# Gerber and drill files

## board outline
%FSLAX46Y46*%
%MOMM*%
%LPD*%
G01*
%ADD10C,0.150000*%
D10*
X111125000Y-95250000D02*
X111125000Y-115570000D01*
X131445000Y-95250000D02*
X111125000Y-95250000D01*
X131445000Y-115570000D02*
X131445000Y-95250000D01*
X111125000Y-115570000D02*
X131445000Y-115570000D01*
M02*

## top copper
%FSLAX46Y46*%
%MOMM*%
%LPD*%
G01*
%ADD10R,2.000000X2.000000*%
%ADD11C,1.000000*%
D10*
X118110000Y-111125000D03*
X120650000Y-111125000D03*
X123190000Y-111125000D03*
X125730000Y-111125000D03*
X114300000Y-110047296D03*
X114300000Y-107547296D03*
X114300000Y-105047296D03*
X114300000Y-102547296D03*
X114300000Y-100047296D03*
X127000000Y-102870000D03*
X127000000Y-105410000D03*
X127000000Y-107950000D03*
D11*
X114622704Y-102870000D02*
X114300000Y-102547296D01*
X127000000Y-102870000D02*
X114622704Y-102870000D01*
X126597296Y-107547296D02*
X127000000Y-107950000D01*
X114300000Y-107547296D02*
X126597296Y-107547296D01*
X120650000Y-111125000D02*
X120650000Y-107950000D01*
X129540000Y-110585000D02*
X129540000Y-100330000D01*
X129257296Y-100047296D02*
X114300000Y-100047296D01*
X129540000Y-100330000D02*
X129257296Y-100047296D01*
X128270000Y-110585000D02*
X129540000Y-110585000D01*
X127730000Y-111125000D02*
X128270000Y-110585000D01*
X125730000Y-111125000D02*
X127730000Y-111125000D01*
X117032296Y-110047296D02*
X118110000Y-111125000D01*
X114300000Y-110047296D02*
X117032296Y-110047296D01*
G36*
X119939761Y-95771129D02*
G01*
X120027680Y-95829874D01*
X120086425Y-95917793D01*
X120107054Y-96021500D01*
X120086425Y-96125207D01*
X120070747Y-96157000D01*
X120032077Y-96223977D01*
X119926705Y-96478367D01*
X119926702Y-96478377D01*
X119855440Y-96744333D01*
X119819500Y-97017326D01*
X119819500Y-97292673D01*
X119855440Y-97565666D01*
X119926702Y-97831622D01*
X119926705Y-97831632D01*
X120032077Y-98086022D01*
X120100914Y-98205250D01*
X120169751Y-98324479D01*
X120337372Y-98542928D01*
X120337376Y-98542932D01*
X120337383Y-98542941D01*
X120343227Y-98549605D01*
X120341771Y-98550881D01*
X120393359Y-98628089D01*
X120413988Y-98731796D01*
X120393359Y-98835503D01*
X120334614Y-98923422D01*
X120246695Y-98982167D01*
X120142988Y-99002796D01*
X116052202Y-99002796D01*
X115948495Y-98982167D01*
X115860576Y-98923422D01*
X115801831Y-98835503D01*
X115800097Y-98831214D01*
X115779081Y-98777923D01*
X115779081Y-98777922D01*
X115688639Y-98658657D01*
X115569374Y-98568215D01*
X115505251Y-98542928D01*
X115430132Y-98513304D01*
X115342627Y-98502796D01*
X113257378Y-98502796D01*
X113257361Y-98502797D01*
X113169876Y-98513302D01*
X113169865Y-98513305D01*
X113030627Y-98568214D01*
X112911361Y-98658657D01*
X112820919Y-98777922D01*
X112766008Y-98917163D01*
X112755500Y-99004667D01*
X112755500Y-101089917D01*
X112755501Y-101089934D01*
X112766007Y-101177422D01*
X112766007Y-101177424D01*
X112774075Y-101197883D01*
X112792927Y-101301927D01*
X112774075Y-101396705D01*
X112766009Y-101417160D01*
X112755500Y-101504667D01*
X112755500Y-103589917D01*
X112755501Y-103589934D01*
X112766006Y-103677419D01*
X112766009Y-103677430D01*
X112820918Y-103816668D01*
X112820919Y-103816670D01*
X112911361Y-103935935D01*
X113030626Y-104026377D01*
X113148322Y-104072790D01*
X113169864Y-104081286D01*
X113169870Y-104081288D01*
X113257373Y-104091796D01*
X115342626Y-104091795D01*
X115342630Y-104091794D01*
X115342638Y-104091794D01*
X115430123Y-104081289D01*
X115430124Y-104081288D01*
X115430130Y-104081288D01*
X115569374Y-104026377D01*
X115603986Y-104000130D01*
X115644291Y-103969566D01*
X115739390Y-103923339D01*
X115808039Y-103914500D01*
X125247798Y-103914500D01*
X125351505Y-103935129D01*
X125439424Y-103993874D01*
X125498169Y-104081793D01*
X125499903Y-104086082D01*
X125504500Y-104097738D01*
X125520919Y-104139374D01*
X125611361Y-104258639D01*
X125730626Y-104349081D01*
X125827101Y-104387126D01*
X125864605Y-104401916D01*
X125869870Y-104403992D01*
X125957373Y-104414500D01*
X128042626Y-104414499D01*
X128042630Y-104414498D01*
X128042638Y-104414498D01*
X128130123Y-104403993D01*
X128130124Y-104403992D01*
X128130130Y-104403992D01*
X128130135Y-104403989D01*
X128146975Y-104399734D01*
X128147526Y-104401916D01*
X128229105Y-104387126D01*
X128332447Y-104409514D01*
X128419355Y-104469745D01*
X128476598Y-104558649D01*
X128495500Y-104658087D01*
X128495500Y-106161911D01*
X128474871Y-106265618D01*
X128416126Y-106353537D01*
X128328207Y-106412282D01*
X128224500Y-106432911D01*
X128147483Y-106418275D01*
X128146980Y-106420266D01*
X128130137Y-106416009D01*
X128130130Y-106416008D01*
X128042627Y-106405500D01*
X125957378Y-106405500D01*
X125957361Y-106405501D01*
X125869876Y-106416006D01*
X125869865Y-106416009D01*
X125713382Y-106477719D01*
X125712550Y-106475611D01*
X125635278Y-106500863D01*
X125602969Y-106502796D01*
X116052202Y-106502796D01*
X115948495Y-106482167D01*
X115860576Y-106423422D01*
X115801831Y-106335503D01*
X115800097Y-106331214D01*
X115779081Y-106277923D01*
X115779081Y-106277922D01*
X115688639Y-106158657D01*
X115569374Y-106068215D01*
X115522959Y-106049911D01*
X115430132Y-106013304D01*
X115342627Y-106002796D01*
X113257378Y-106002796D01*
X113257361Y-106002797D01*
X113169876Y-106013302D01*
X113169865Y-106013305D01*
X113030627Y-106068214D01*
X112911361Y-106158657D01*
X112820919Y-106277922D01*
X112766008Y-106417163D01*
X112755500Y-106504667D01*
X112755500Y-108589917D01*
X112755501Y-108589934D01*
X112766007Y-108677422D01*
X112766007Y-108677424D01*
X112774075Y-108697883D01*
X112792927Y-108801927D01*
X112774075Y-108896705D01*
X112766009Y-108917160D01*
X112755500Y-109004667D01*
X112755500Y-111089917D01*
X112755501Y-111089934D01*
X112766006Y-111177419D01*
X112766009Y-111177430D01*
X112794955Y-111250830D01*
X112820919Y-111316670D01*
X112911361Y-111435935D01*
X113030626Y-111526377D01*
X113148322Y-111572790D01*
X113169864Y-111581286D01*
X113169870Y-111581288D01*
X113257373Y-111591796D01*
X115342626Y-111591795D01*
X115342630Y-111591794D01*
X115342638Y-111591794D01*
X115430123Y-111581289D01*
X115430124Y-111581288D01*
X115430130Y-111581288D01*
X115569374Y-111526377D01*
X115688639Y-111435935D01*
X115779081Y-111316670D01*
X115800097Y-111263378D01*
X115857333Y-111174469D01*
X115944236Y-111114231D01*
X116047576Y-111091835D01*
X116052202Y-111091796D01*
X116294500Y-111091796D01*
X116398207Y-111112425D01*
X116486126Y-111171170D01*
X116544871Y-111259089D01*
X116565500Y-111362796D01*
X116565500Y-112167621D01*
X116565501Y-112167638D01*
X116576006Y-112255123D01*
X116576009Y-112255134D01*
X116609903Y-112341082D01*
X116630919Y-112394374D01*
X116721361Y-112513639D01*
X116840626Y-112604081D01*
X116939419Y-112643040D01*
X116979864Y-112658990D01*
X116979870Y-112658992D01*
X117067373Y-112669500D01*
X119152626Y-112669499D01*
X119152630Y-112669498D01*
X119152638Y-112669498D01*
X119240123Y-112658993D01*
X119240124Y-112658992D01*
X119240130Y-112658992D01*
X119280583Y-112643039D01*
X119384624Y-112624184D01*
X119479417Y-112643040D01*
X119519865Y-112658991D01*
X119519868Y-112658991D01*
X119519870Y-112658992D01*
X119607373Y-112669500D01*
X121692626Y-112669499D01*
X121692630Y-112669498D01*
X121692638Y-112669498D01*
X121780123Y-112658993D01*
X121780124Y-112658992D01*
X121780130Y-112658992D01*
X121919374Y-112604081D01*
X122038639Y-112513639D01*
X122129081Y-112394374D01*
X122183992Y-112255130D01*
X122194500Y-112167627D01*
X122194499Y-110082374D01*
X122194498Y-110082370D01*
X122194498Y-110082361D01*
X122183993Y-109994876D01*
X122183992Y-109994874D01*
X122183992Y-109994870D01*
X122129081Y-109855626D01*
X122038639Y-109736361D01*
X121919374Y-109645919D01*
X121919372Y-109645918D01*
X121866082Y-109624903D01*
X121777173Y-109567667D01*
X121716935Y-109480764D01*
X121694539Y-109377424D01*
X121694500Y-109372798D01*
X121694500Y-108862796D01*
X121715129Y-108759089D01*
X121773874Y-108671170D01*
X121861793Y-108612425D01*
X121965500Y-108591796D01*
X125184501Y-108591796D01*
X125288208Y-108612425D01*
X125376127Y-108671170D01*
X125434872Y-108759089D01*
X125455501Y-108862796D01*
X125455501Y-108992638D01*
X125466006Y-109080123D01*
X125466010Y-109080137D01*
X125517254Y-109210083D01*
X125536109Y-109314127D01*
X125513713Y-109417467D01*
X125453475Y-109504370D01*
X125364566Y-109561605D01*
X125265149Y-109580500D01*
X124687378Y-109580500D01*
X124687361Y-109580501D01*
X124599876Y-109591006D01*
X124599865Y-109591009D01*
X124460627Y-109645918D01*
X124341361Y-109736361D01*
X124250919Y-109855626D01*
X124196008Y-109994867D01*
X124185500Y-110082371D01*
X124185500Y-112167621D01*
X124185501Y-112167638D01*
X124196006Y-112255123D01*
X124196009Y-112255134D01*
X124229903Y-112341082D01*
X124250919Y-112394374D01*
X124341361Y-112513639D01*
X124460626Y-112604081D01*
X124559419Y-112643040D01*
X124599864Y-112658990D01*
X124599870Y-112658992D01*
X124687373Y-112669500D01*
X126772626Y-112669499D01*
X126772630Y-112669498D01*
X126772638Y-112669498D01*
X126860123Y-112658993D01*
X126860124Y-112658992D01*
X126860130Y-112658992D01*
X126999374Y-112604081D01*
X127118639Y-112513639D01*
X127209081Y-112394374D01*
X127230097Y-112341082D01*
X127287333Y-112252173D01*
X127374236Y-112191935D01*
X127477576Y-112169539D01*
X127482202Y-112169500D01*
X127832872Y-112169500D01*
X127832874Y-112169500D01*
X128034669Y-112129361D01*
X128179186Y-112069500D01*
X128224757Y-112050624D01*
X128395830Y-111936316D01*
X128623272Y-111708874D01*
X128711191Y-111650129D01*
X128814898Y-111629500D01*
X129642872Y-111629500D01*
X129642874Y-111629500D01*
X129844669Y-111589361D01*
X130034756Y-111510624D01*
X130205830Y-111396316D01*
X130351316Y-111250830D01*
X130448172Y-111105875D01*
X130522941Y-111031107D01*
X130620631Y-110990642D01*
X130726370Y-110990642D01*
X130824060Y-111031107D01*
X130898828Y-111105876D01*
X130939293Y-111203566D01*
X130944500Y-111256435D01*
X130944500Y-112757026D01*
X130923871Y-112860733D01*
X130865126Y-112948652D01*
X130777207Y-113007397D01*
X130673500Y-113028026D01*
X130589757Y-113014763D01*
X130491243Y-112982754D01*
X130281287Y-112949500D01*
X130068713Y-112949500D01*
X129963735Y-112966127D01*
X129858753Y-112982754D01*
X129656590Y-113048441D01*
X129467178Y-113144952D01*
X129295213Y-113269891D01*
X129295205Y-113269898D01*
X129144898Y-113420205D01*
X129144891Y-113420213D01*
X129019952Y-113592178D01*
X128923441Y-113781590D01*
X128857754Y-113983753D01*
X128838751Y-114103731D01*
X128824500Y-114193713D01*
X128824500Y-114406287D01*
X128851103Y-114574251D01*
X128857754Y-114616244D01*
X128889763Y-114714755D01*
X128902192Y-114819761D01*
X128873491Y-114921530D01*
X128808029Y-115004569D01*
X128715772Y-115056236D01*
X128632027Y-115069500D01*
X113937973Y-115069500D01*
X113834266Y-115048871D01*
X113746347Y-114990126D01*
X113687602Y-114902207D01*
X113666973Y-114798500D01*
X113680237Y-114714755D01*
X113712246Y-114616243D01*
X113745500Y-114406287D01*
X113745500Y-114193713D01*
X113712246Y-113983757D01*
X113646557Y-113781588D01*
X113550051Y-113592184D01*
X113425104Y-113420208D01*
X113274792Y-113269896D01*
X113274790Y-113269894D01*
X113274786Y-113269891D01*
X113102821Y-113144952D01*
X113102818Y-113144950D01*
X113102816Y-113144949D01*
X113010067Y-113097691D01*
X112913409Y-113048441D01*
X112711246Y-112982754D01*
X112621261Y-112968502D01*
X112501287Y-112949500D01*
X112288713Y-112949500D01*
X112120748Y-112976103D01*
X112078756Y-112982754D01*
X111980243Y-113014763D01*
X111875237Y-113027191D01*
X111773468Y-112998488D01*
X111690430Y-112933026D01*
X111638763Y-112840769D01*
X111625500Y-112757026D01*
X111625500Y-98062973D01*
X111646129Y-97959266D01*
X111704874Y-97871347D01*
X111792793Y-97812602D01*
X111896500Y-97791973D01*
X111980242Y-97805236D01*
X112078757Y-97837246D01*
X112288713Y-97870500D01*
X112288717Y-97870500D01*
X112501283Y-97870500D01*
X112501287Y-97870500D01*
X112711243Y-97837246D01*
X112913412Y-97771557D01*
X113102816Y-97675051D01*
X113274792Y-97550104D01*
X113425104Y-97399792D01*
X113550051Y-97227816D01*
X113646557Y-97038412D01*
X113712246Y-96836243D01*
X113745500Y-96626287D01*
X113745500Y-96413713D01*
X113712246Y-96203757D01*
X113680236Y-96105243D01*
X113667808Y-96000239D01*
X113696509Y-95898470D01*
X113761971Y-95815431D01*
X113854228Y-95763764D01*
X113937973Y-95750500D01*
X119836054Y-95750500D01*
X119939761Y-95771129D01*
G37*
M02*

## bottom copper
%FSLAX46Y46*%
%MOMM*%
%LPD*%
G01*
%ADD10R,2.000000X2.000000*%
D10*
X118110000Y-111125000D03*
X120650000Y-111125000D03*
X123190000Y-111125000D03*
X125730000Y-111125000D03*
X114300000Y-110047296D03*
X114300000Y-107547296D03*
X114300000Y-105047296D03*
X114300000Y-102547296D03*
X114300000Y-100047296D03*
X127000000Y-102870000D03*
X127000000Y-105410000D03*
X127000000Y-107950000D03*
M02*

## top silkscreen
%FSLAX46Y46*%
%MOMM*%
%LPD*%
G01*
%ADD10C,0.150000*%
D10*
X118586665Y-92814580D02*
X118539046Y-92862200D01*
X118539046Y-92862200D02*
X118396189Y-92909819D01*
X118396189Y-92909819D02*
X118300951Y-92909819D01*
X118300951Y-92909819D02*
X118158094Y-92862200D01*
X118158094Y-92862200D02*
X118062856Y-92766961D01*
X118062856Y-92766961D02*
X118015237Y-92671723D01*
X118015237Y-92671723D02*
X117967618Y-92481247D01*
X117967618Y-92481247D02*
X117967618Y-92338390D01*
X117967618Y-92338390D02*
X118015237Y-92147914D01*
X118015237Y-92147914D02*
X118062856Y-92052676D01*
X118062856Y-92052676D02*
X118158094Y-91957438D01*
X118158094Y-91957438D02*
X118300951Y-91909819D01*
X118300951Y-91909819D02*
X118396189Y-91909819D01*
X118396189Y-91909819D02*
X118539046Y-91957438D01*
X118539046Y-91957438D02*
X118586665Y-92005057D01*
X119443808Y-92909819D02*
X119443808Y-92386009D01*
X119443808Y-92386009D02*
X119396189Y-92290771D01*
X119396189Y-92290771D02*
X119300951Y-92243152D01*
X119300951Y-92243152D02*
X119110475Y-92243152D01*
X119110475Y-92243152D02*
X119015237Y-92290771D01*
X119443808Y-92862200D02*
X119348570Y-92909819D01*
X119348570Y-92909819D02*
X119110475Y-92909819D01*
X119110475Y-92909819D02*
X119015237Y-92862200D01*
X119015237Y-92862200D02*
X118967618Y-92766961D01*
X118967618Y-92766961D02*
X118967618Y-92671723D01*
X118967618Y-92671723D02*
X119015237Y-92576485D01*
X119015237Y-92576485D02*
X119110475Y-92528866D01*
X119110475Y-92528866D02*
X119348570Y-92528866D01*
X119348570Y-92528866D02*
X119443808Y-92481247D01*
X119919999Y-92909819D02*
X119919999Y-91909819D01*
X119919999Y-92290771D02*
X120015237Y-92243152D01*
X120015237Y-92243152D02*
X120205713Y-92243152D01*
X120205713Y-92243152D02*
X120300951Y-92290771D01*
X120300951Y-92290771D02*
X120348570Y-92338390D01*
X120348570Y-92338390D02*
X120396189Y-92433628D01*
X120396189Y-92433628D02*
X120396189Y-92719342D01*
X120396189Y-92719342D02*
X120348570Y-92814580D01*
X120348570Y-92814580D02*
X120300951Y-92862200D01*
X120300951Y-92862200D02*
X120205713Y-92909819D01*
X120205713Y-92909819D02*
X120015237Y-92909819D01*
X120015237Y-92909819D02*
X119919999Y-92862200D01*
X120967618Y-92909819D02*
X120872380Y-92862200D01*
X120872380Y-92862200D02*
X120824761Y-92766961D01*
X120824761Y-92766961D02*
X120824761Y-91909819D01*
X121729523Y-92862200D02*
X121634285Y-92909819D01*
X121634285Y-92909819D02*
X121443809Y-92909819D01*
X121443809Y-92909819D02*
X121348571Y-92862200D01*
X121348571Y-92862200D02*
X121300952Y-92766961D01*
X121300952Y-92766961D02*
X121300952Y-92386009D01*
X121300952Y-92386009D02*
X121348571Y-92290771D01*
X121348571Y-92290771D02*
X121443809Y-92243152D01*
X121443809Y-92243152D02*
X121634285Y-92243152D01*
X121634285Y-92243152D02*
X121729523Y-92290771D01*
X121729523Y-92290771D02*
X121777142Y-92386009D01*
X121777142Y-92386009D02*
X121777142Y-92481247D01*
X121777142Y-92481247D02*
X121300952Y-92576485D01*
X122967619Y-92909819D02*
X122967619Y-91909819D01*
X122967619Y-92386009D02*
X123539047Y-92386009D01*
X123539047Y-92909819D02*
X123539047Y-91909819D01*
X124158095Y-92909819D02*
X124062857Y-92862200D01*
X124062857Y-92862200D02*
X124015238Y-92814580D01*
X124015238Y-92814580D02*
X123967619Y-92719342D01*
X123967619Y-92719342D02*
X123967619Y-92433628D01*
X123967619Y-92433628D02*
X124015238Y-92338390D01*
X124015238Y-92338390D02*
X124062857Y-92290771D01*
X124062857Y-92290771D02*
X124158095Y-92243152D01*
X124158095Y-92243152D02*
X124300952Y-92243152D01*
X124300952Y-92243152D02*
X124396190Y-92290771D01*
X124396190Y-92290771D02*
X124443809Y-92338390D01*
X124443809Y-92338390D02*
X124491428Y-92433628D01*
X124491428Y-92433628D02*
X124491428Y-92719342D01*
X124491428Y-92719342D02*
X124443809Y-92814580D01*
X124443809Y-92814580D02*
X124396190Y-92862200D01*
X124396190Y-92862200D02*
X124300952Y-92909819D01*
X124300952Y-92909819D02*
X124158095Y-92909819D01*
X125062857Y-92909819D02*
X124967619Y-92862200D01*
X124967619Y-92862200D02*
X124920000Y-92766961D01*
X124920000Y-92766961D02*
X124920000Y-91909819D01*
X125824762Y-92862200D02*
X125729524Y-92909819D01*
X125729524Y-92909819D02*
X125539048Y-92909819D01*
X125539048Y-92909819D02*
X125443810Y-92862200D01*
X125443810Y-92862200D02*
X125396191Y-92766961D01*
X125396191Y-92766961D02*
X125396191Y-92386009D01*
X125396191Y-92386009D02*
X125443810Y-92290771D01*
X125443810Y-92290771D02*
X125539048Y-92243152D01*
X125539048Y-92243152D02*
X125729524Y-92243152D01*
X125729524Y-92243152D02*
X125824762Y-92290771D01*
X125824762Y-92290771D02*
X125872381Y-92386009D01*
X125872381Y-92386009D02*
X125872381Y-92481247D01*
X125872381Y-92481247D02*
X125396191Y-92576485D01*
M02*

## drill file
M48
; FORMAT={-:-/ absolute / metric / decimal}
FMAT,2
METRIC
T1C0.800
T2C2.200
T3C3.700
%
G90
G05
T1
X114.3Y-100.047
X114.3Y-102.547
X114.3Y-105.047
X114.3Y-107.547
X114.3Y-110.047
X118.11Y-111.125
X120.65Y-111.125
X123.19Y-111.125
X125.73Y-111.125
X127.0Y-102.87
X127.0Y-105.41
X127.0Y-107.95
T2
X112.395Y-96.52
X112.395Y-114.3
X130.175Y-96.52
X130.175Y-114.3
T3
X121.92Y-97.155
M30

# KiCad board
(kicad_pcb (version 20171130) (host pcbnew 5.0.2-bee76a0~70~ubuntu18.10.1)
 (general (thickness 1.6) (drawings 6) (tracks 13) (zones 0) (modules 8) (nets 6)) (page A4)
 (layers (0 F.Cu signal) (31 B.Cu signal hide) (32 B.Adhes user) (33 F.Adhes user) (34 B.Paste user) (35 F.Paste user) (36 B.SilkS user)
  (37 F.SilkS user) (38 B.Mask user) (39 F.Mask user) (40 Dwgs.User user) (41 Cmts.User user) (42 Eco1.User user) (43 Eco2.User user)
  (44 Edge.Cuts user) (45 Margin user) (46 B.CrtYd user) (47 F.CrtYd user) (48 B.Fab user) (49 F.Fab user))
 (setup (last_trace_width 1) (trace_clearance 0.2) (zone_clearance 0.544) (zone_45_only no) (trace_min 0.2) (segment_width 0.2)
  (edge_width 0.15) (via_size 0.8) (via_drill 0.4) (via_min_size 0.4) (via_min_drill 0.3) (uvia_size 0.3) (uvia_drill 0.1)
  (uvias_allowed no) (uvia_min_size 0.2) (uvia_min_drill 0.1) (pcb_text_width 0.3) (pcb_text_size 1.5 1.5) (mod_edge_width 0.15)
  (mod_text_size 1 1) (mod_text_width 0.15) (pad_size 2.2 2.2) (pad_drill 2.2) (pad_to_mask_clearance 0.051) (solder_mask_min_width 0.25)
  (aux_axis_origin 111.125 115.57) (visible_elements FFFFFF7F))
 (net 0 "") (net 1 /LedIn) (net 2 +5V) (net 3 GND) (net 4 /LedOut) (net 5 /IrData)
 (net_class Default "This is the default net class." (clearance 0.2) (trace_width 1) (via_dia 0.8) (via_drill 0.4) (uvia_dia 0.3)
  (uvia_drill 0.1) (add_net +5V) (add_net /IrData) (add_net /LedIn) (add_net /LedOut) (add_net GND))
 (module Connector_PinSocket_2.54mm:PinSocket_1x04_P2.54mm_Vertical (layer B.Cu) (at 118.11 111.125 270)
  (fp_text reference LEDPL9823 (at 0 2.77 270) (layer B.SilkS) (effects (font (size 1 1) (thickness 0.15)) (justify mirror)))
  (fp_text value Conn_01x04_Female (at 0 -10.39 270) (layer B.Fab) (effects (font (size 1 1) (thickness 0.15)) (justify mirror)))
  (pad 1 thru_hole rect (at 0 0 270) (size 2 2) (drill 0.8) (layers *.Cu *.Mask) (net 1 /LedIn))
  (pad 2 thru_hole rect (at 0 -2.54 270) (size 2 2) (drill 0.8) (layers *.Cu *.Mask) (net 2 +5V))
  (pad 3 thru_hole rect (at 0 -5.08 270) (size 2 2) (drill 0.8) (layers *.Cu *.Mask) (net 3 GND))
  (pad 4 thru_hole rect (at 0 -7.62 270) (size 2 2) (drill 0.8) (layers *.Cu *.Mask) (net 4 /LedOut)))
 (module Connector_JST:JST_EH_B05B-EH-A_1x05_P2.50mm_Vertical (layer B.Cu) (at 114.3 110.047296 90)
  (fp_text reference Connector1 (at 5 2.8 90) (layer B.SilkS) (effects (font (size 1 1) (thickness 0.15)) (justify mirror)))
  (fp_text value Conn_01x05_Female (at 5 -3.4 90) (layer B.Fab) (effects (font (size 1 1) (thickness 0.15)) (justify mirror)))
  (pad 1 thru_hole rect (at 0 0 90) (size 2 2) (drill 0.8) (layers *.Cu *.Mask) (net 1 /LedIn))
  (pad 2 thru_hole rect (at 2.5 0 90) (size 2 2) (drill 0.8) (layers *.Cu *.Mask) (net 2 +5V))
  (pad 3 thru_hole rect (at 5 0 90) (size 2 2) (drill 0.8) (layers *.Cu *.Mask) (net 3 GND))
  (pad 4 thru_hole rect (at 7.5 0 90) (size 2 2) (drill 0.8) (layers *.Cu *.Mask) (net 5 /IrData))
  (pad 5 thru_hole rect (at 10 0 90) (size 2 2) (drill 0.8) (layers *.Cu *.Mask) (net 4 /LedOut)))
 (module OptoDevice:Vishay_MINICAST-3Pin (layer B.Cu) (at 127 102.87 270)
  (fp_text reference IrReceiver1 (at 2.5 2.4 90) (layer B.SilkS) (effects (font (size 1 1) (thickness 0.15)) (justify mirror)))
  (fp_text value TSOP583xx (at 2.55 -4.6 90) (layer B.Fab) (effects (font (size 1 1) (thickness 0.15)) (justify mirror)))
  (pad 1 thru_hole rect (at 0 0 270) (size 2 2) (drill 0.8) (layers *.Cu *.Mask) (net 5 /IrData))
  (pad 2 thru_hole rect (at 2.54 0 270) (size 2 2) (drill 0.8) (layers *.Cu *.Mask) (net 3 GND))
  (pad 3 thru_hole rect (at 5.08 0 270) (size 2 2) (drill 0.8) (layers *.Cu *.Mask) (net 2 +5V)))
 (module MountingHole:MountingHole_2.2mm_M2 (layer F.Cu) (at 112.395 96.52)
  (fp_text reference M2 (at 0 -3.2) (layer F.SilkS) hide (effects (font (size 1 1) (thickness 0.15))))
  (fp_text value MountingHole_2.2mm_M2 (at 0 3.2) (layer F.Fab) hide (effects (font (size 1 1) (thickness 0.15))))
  (pad "" np_thru_hole circle (at 0 0) (size 2.2 2.2) (drill 2.2) (layers *.Cu *.Mask)))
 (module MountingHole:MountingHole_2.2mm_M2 (layer F.Cu) (at 112.395 114.3)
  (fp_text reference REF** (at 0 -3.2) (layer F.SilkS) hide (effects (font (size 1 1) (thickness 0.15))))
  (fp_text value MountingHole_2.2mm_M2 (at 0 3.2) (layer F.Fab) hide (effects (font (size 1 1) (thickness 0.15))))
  (pad 1 np_thru_hole circle (at 0 0) (size 2.2 2.2) (drill 2.2) (layers *.Cu *.Mask)))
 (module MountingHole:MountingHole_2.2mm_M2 (layer F.Cu) (at 130.175 114.3)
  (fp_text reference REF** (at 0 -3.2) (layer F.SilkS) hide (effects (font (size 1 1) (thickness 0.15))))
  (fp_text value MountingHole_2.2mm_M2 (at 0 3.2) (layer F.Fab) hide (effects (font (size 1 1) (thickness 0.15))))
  (pad 1 np_thru_hole circle (at 0 0) (size 2.2 2.2) (drill 2.2) (layers *.Cu *.Mask)))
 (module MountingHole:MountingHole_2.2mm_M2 (layer F.Cu) (at 130.175 96.52)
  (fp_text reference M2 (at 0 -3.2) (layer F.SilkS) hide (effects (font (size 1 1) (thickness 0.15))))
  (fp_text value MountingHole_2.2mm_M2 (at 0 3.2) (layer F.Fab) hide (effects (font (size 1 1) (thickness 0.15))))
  (pad 1 np_thru_hole circle (at 0 0) (size 2.2 2.2) (drill 2.2) (layers *.Cu *.Mask)))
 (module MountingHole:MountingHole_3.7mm (layer F.Cu) (at 121.92 97.155)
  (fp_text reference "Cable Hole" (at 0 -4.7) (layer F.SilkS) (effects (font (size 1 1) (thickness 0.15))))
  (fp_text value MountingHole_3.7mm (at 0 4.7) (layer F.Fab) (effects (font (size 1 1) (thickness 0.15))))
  (pad 1 np_thru_hole circle (at 0 0) (size 3.7 3.7) (drill 3.7) (layers *.Cu *.Mask)))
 (gr_line (start 111.125 95.25) (end 111.125 115.57) (layer Edge.Cuts) (width 0.15))
 (gr_line (start 131.445 95.25) (end 111.125 95.25) (layer Edge.Cuts) (width 0.15))
 (gr_line (start 131.445 115.57) (end 131.445 95.25) (layer Edge.Cuts) (width 0.15))
 (gr_line (start 111.125 115.57) (end 131.445 115.57) (layer Edge.Cuts) (width 0.15))
 (segment (start 114.622704 102.87) (end 114.3 102.547296) (width 1) (layer F.Cu) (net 5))
 (segment (start 127 102.87) (end 114.622704 102.87) (width 1) (layer F.Cu) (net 5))
 (segment (start 126.597296 107.547296) (end 127 107.95) (width 1) (layer F.Cu) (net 2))
 (segment (start 114.3 107.547296) (end 126.597296 107.547296) (width 1) (layer F.Cu) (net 2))
 (segment (start 120.65 111.125) (end 120.65 107.95) (width 1) (layer F.Cu) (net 2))
 (segment (start 129.54 110.585) (end 129.54 100.33) (width 1) (layer F.Cu) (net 4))
 (segment (start 129.257296 100.047296) (end 114.3 100.047296) (width 1) (layer F.Cu) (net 4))
 (segment (start 129.54 100.33) (end 129.257296 100.047296) (width 1) (layer F.Cu) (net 4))
 (segment (start 128.27 110.585) (end 129.54 110.585) (width 1) (layer F.Cu) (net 4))
 (segment (start 127.73 111.125) (end 128.27 110.585) (width 1) (layer F.Cu) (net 4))
 (segment (start 125.73 111.125) (end 127.73 111.125) (width 1) (layer F.Cu) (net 4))
 (segment (start 117.032296 110.047296) (end 118.11 111.125) (width 1) (layer F.Cu) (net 1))
 (segment (start 114.3 110.047296) (end 117.032296 110.047296) (width 1) (layer F.Cu) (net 1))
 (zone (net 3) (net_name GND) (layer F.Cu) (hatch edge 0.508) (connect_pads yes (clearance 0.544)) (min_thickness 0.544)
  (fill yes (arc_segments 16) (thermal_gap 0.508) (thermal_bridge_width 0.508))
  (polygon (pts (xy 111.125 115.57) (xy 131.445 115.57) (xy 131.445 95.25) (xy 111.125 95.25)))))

